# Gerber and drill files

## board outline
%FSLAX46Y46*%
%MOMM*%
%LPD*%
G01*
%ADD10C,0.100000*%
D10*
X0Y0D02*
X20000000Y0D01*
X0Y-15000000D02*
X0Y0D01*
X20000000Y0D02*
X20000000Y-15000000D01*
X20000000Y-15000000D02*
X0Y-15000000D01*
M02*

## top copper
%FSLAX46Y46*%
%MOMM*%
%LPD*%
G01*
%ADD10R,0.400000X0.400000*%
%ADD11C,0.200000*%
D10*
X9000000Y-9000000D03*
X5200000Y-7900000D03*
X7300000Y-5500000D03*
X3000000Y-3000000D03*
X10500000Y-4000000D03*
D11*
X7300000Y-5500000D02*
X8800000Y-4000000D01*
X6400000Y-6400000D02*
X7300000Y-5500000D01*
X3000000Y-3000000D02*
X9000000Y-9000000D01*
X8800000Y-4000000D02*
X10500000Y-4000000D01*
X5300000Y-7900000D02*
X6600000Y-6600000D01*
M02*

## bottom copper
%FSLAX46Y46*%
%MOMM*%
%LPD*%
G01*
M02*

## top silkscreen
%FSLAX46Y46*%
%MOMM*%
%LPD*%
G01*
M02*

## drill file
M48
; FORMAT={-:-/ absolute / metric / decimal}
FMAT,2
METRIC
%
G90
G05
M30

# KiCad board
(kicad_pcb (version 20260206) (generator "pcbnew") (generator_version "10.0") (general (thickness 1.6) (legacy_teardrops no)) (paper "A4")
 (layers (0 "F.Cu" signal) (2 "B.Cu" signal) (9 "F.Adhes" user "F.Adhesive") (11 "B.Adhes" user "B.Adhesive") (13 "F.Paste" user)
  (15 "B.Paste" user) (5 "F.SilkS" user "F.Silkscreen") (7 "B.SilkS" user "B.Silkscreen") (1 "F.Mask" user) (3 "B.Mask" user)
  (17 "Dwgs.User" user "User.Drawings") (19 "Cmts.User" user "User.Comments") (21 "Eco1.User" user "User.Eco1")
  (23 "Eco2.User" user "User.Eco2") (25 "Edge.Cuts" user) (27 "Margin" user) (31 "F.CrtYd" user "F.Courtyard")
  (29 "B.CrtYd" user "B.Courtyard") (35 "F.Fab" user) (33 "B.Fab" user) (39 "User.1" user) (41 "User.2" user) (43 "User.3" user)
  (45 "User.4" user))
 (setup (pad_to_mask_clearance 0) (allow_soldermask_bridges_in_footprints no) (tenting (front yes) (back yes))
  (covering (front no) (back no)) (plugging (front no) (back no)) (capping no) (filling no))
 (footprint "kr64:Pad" (layer "F.Cu") (at 9 9)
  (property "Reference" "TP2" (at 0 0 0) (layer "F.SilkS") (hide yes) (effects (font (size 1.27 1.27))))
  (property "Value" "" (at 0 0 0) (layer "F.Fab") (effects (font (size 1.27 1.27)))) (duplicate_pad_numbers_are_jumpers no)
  (pad "1" smd rect (at 0 0) (size 0.4 0.4) (layers "F.Cu" "F.Mask" "F.Paste") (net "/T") (thermal_bridge_angle 45)))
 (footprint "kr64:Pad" (layer "F.Cu") (at 5.2 7.9)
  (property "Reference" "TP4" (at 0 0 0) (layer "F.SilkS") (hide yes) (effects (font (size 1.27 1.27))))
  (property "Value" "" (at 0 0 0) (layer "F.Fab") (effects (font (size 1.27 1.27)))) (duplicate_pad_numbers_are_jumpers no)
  (pad "1" smd rect (at 0 0) (size 0.4 0.4) (layers "F.Cu" "F.Mask" "F.Paste") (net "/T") (thermal_bridge_angle 45)))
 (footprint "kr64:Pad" (layer "F.Cu") (at 7.3 5.5)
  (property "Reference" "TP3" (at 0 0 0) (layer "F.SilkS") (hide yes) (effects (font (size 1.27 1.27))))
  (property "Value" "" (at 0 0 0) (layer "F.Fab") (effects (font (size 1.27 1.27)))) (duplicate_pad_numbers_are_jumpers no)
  (pad "1" smd rect (at 0 0) (size 0.4 0.4) (layers "F.Cu" "F.Mask" "F.Paste") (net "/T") (thermal_bridge_angle 45)))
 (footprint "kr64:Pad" (layer "F.Cu") (at 3 3)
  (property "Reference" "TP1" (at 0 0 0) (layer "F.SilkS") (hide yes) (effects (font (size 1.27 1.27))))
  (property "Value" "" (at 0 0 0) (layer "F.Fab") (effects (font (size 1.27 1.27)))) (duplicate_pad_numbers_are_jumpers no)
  (pad "1" smd rect (at 0 0) (size 0.4 0.4) (layers "F.Cu" "F.Mask" "F.Paste") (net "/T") (thermal_bridge_angle 45)))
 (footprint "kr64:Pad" (layer "F.Cu") (at 10.5 4)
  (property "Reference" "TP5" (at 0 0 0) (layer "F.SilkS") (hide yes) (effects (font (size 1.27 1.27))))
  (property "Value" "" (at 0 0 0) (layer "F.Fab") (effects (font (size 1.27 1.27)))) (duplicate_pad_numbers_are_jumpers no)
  (pad "1" smd rect (at 0 0) (size 0.4 0.4) (layers "F.Cu" "F.Mask" "F.Paste") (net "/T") (thermal_bridge_angle 45)))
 (gr_line (start 0 0) (end 20 0) (stroke (width 0.1) (type default)) (layer "Edge.Cuts"))
 (gr_line (start 0 15) (end 0 0) (stroke (width 0.1) (type default)) (layer "Edge.Cuts"))
 (gr_line (start 20 0) (end 20 15) (stroke (width 0.1) (type default)) (layer "Edge.Cuts"))
 (gr_line (start 20 15) (end 0 15) (stroke (width 0.1) (type default)) (layer "Edge.Cuts"))
 (segment (start 7.3 5.5) (end 8.8 4) (width 0.2) (layer "F.Cu") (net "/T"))
 (segment (start 6.4 6.4) (end 7.3 5.5) (width 0.2) (layer "F.Cu") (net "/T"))
 (segment (start 3 3) (end 9 9) (width 0.2) (layer "F.Cu") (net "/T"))
 (segment (start 8.8 4) (end 10.5 4) (width 0.2) (layer "F.Cu") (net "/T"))
 (segment (start 5.3 7.9) (end 6.6 6.6) (width 0.2) (layer "F.Cu") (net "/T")))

